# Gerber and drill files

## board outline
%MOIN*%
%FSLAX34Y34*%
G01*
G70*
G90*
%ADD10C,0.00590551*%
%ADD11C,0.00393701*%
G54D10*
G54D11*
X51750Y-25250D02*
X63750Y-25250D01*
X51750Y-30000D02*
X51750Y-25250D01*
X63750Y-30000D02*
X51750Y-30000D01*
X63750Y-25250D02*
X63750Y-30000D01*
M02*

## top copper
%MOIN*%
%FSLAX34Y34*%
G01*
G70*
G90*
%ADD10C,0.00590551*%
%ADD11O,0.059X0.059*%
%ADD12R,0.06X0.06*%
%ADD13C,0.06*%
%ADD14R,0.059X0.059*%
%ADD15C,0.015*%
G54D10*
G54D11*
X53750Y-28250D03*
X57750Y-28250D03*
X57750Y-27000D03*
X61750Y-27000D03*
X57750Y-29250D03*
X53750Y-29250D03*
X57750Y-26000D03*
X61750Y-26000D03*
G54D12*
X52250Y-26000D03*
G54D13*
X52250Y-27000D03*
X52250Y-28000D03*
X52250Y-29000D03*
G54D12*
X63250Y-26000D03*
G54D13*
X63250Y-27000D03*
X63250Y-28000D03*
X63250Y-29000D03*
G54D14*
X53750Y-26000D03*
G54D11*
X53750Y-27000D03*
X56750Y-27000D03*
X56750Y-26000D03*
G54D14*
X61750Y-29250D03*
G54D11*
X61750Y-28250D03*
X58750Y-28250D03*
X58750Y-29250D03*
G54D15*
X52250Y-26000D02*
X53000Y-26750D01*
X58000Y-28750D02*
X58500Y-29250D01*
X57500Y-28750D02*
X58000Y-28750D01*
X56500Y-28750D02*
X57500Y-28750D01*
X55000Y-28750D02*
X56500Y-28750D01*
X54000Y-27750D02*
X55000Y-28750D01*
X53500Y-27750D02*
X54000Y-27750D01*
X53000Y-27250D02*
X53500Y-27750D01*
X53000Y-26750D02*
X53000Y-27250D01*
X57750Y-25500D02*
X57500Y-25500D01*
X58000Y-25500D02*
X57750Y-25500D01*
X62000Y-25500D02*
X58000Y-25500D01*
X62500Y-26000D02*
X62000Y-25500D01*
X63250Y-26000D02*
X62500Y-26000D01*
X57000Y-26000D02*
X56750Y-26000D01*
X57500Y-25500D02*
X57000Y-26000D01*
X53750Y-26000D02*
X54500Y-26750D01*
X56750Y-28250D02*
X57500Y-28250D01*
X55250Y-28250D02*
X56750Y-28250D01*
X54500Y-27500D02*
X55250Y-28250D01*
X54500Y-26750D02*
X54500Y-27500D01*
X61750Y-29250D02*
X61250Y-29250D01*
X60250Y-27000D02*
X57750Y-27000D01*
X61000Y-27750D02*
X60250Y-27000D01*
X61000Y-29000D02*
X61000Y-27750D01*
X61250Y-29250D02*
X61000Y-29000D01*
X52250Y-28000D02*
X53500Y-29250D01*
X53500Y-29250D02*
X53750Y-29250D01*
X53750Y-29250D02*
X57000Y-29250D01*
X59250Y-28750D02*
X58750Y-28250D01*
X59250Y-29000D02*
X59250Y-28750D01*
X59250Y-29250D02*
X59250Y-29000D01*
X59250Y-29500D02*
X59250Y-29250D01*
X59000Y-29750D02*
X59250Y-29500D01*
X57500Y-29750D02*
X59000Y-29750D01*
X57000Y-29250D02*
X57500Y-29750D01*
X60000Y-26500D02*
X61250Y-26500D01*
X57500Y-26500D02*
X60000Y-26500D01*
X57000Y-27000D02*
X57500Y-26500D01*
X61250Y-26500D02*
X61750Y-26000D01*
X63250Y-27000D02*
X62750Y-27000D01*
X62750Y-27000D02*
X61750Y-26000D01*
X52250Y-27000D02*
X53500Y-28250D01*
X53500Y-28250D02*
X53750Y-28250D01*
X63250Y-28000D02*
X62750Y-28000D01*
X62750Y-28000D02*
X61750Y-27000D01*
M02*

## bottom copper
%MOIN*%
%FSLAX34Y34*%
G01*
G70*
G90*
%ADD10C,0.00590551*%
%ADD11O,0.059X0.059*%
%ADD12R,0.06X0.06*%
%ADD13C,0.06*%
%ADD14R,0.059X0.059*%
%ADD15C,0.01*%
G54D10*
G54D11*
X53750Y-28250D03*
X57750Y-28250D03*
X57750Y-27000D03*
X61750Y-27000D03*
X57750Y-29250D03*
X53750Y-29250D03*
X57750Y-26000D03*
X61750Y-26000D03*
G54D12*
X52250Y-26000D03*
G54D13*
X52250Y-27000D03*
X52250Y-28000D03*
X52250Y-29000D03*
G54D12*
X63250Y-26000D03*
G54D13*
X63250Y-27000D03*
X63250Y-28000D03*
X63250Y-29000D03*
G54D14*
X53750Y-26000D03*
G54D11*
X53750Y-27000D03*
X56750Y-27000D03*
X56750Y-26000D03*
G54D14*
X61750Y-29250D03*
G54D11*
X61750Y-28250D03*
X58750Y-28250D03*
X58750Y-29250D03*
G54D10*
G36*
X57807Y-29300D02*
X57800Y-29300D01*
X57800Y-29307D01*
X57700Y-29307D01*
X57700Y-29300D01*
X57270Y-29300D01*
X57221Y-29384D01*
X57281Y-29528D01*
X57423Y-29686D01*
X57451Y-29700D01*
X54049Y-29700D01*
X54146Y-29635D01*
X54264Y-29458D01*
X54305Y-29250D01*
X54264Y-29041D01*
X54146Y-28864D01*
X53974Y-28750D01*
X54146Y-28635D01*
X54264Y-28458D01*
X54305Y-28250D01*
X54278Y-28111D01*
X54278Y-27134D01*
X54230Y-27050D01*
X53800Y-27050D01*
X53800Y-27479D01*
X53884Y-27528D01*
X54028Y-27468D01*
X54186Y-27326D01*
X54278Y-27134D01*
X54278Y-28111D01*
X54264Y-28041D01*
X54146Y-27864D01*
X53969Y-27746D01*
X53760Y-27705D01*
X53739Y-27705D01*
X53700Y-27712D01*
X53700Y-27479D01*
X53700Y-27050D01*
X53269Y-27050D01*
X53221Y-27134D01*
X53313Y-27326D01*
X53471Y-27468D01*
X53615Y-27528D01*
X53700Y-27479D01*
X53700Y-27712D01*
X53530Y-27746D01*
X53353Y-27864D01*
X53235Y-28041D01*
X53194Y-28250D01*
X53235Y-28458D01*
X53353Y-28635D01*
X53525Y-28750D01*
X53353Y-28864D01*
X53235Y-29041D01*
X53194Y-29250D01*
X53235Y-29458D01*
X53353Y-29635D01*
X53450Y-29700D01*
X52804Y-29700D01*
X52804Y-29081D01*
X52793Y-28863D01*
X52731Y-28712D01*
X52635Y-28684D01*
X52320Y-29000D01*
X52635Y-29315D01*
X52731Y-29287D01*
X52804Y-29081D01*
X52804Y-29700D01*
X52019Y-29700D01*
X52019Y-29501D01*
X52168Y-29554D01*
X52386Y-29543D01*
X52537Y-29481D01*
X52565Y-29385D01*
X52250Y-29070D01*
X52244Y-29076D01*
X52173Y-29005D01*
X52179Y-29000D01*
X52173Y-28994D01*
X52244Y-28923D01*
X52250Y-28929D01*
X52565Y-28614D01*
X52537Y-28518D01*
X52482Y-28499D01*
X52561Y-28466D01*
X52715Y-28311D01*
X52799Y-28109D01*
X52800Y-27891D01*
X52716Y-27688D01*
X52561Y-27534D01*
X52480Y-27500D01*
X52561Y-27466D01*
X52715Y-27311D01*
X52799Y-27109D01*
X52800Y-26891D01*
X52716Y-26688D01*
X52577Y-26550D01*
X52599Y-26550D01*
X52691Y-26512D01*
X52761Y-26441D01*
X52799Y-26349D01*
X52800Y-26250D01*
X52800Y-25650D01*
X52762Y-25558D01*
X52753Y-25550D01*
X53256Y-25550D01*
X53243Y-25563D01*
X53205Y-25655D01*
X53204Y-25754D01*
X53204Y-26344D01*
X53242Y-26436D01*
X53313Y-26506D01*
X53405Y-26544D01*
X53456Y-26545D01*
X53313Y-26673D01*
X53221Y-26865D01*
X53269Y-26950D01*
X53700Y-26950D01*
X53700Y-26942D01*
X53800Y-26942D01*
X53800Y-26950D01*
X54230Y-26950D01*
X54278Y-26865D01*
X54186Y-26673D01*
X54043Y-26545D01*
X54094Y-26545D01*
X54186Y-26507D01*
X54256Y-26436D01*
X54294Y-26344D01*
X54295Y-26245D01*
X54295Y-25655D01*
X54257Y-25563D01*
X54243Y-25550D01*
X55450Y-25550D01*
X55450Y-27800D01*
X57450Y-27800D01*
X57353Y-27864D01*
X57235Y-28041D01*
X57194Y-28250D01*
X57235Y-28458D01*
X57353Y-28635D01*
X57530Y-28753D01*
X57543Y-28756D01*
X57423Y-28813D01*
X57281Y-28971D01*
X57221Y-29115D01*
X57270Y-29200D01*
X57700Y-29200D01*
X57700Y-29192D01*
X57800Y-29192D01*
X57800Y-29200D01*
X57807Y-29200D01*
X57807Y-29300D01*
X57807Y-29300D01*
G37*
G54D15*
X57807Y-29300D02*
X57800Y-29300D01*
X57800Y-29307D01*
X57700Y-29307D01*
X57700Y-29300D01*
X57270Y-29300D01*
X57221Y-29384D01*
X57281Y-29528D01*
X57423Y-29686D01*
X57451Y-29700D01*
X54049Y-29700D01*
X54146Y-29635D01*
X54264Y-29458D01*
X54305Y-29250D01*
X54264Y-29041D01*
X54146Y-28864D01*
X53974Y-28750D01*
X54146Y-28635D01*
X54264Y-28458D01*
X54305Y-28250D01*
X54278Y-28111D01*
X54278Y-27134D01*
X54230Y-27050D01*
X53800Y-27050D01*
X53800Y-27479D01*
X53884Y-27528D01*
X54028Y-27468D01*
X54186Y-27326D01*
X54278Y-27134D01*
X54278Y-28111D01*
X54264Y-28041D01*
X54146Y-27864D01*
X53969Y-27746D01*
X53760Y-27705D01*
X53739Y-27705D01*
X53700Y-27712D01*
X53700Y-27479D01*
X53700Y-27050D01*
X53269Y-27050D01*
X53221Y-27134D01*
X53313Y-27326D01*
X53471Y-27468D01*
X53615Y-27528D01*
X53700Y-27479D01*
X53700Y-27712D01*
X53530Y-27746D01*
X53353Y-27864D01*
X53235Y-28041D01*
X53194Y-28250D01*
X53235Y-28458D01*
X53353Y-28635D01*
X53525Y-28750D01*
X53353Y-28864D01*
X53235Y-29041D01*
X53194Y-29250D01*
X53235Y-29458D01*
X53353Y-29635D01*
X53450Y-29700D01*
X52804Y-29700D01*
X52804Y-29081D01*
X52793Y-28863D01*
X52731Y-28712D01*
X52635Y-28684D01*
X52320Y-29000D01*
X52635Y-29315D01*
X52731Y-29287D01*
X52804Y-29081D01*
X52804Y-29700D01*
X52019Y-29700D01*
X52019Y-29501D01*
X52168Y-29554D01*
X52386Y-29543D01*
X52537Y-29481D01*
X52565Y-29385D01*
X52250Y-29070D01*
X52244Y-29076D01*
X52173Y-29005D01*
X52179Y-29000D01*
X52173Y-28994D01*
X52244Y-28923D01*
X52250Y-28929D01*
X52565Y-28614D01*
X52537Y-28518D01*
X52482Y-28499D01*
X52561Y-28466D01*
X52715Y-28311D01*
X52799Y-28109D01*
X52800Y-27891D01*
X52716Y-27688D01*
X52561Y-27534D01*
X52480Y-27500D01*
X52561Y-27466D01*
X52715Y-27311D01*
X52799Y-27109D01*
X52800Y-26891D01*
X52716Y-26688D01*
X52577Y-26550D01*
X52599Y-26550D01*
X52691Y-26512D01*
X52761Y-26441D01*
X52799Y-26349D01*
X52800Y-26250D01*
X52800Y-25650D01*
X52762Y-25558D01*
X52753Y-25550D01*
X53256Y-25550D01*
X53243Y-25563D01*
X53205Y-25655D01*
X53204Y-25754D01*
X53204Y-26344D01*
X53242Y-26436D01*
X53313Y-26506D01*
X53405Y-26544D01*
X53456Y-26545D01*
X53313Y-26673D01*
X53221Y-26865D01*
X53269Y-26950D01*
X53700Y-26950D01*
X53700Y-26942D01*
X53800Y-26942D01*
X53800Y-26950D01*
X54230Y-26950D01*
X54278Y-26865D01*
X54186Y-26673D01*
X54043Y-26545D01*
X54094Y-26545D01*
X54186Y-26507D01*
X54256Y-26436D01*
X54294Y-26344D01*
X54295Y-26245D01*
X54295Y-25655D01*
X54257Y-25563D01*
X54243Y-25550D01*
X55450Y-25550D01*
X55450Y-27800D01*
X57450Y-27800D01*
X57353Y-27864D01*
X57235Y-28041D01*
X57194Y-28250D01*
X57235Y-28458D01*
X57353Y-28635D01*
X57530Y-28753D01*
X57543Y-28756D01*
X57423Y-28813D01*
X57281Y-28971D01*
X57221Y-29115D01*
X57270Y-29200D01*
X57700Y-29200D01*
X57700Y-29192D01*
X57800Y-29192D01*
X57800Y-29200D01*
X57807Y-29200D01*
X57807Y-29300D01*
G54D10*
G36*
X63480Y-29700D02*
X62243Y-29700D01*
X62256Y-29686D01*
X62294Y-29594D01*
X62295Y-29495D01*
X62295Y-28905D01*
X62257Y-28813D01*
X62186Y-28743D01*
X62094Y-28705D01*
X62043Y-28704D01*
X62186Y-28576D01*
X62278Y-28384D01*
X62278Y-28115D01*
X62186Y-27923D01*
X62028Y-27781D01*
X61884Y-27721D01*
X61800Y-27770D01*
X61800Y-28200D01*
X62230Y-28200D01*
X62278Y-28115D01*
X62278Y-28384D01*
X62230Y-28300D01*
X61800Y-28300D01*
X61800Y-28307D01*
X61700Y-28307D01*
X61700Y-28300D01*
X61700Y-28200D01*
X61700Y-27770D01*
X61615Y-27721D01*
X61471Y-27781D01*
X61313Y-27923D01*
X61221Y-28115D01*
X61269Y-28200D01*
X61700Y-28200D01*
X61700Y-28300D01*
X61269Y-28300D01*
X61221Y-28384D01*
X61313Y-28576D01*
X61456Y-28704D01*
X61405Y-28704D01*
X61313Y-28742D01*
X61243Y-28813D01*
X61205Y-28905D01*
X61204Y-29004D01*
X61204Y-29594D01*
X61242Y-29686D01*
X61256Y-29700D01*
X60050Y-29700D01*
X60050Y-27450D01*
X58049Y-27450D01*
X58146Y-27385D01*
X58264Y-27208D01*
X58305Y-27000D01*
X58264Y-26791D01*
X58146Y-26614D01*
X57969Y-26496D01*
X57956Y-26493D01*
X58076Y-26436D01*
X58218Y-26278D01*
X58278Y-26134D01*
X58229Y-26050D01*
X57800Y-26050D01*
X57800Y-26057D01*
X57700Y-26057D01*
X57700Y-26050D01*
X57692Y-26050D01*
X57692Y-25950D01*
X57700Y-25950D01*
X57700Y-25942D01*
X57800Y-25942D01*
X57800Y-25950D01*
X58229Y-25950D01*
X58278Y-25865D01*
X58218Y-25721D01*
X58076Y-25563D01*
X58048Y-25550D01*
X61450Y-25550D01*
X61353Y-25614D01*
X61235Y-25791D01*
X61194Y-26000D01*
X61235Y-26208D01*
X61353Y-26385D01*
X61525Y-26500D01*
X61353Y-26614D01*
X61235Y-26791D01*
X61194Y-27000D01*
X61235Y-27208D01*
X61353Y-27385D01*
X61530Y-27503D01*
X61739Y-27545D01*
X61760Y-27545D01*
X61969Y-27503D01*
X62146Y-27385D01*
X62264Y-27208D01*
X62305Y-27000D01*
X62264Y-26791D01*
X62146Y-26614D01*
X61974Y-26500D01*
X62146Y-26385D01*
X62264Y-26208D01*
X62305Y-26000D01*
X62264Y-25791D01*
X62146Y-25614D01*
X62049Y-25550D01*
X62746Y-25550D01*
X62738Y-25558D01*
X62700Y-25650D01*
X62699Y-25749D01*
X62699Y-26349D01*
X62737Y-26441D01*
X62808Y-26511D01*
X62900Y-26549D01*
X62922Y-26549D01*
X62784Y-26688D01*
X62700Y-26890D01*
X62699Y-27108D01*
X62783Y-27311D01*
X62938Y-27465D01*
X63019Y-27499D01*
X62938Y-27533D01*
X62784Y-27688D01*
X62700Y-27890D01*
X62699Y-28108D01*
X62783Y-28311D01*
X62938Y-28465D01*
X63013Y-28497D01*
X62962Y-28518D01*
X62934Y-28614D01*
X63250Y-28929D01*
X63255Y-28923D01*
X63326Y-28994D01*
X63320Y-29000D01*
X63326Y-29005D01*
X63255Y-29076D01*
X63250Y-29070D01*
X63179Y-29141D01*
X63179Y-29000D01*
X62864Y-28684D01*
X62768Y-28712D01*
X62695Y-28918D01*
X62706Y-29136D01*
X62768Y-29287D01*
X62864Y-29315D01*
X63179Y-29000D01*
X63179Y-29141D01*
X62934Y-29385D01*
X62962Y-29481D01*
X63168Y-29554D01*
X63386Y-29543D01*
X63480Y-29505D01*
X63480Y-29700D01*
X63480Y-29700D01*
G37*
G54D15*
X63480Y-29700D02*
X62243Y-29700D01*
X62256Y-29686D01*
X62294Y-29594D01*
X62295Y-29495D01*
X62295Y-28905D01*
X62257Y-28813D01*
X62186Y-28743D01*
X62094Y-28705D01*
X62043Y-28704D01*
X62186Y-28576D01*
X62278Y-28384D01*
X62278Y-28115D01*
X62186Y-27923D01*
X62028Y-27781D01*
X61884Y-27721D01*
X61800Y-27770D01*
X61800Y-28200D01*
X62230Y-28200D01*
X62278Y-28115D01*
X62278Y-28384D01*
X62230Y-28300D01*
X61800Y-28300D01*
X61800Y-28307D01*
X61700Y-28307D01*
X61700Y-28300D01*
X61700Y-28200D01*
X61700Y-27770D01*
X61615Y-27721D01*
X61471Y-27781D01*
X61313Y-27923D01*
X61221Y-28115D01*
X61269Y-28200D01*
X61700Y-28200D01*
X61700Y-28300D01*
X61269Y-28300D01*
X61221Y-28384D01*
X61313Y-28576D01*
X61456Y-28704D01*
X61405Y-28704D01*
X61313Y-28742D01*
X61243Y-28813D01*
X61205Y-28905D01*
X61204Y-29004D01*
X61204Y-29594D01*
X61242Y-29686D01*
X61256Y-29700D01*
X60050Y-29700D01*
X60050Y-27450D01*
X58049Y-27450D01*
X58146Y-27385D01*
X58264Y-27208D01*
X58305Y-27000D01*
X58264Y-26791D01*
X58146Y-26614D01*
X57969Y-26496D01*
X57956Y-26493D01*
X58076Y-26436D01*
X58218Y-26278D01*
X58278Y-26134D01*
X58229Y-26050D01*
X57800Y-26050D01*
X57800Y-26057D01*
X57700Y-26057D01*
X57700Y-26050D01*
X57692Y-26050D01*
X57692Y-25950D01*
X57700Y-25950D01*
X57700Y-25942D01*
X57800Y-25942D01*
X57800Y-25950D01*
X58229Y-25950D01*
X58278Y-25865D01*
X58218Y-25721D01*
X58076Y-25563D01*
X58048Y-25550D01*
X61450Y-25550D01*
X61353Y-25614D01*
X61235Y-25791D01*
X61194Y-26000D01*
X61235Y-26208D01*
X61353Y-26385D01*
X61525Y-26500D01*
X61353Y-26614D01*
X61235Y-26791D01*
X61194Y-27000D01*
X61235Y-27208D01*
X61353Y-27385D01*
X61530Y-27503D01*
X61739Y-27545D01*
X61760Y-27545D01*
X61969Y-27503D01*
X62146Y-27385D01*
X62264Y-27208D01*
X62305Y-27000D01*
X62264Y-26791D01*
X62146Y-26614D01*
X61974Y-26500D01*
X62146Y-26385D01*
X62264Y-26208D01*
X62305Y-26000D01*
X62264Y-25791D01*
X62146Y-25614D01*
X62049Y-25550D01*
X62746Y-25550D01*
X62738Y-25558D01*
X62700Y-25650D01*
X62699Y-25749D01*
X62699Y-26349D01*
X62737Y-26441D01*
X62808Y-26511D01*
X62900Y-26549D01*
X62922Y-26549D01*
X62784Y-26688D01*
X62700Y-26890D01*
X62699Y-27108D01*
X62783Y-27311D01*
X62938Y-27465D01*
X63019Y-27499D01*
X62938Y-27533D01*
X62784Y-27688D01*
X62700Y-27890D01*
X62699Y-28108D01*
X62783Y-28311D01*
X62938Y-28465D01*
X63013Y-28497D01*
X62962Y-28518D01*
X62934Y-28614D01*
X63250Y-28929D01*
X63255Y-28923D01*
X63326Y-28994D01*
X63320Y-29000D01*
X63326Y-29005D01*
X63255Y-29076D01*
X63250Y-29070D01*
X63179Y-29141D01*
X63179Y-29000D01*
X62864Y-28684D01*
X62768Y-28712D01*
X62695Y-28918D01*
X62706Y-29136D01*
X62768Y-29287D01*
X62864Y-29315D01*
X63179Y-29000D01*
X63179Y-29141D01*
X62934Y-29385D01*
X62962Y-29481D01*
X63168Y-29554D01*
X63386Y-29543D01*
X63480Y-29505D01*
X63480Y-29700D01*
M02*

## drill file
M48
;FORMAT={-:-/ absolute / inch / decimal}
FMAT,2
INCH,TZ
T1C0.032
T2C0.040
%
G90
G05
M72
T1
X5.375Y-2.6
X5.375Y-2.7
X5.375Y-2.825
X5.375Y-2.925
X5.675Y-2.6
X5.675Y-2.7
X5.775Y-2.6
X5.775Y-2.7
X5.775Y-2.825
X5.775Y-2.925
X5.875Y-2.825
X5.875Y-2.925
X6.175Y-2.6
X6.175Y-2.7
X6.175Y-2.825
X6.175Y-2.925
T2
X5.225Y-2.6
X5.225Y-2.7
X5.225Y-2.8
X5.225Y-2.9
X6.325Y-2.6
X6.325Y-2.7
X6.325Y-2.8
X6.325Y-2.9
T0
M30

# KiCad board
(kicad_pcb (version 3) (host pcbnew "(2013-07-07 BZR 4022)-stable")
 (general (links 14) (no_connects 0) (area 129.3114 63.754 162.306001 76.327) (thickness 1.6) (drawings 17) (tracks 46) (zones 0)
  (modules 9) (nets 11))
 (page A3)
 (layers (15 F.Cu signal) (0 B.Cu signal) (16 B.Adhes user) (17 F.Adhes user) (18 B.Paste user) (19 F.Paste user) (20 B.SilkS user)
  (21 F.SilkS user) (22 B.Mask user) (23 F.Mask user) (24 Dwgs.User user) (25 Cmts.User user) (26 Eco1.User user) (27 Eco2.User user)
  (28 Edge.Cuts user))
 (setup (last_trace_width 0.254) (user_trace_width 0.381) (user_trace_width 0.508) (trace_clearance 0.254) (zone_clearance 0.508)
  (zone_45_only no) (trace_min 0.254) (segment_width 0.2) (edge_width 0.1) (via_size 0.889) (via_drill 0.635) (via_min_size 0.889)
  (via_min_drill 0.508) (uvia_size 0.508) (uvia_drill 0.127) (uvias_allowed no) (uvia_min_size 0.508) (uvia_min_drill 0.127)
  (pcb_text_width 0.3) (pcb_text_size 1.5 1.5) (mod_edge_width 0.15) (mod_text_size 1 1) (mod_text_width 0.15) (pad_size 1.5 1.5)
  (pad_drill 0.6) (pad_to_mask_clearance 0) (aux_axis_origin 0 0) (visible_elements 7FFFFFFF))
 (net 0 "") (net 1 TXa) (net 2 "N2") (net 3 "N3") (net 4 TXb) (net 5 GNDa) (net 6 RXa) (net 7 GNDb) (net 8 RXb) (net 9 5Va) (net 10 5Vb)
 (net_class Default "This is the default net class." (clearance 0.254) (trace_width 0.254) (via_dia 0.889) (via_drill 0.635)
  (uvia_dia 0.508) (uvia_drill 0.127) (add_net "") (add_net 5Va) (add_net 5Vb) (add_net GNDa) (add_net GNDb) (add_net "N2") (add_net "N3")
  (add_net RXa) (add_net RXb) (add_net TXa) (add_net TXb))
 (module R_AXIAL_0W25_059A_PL (layer F.Cu) (at 136.525 71.755) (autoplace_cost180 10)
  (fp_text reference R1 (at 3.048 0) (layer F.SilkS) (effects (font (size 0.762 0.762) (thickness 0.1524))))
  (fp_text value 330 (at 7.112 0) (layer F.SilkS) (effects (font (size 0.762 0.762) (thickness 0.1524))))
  (pad 1 thru_hole oval (at 0 0) (size 1.4986 1.4986) (drill 0.8128) (layers *.Cu *.Mask F.SilkS) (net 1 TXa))
  (pad 2 thru_hole oval (at 10.16 0) (size 1.4986 1.4986) (drill 0.8128) (layers *.Cu *.Mask F.SilkS) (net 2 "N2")))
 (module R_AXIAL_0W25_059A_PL (layer F.Cu) (at 146.685 68.58) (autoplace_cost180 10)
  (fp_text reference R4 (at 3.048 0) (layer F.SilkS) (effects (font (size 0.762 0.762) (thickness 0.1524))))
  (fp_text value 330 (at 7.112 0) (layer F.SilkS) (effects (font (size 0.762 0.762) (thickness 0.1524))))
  (pad 1 thru_hole oval (at 0 0) (size 1.4986 1.4986) (drill 0.8128) (layers *.Cu *.Mask F.SilkS) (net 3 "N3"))
  (pad 2 thru_hole oval (at 10.16 0) (size 1.4986 1.4986) (drill 0.8128) (layers *.Cu *.Mask F.SilkS) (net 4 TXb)))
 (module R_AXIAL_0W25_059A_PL (layer F.Cu) (at 146.685 74.295 180) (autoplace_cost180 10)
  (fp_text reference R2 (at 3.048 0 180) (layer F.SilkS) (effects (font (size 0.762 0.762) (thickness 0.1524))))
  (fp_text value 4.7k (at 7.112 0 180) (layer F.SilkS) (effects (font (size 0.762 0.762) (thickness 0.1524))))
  (pad 1 thru_hole oval (at 0 0 180) (size 1.4986 1.4986) (drill 0.8128) (layers *.Cu *.Mask F.SilkS) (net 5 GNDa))
  (pad 2 thru_hole oval (at 10.16 0 180) (size 1.4986 1.4986) (drill 0.8128) (layers *.Cu *.Mask F.SilkS) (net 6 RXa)))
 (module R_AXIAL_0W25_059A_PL (layer F.Cu) (at 146.685 66.04) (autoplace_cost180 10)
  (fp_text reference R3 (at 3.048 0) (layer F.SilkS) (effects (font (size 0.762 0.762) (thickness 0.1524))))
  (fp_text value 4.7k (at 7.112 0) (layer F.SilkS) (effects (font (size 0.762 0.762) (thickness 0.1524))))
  (pad 1 thru_hole oval (at 0 0) (size 1.4986 1.4986) (drill 0.8128) (layers *.Cu *.Mask F.SilkS) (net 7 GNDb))
  (pad 2 thru_hole oval (at 10.16 0) (size 1.4986 1.4986) (drill 0.8128) (layers *.Cu *.Mask F.SilkS) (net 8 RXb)))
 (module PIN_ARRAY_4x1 (layer F.Cu) (at 132.715 69.85 270)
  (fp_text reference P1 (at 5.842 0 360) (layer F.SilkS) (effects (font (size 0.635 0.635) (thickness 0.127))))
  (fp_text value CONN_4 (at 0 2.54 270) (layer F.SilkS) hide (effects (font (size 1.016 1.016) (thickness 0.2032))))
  (pad 1 thru_hole rect (at -3.81 0 270) (size 1.524 1.524) (drill 1.016) (layers *.Cu *.Mask F.SilkS) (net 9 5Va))
  (pad 2 thru_hole circle (at -1.27 0 270) (size 1.524 1.524) (drill 1.016) (layers *.Cu *.Mask F.SilkS) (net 1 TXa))
  (pad 3 thru_hole circle (at 1.27 0 270) (size 1.524 1.524) (drill 1.016) (layers *.Cu *.Mask F.SilkS) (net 6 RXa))
  (pad 4 thru_hole circle (at 3.81 0 270) (size 1.524 1.524) (drill 1.016) (layers *.Cu *.Mask F.SilkS) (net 5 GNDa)))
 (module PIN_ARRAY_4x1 (layer F.Cu) (at 160.655 69.85 270)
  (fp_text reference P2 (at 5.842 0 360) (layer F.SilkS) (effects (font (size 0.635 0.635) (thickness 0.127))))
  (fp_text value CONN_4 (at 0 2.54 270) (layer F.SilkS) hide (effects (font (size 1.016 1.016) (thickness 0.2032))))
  (pad 1 thru_hole rect (at -3.81 0 270) (size 1.524 1.524) (drill 1.016) (layers *.Cu *.Mask F.SilkS) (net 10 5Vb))
  (pad 2 thru_hole circle (at -1.27 0 270) (size 1.524 1.524) (drill 1.016) (layers *.Cu *.Mask F.SilkS) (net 8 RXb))
  (pad 3 thru_hole circle (at 1.27 0 270) (size 1.524 1.524) (drill 1.016) (layers *.Cu *.Mask F.SilkS) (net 4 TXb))
  (pad 4 thru_hole circle (at 3.81 0 270) (size 1.524 1.524) (drill 1.016) (layers *.Cu *.Mask F.SilkS) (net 7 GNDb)))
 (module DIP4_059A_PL (layer F.Cu) (at 140.335 67.31 270)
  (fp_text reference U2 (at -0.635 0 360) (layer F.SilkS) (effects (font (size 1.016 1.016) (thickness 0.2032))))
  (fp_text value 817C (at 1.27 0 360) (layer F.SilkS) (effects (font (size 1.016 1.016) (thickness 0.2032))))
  (pad 1 thru_hole rect (at -1.27 3.81 270) (size 1.4986 1.4986) (drill 0.8128) (layers *.Cu *.Mask F.SilkS) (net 2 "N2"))
  (pad 2 thru_hole oval (at 1.27 3.81 270) (size 1.4986 1.4986) (drill 0.8128) (layers *.Cu *.Mask F.SilkS) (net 5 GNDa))
  (pad 3 thru_hole oval (at 1.27 -3.81 270) (size 1.4986 1.4986) (drill 0.8128) (layers *.Cu *.Mask F.SilkS) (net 8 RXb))
  (pad 4 thru_hole oval (at -1.27 -3.81 270) (size 1.4986 1.4986) (drill 0.8128) (layers *.Cu *.Mask F.SilkS) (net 10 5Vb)))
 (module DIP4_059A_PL (layer F.Cu) (at 153.035 73.025 90)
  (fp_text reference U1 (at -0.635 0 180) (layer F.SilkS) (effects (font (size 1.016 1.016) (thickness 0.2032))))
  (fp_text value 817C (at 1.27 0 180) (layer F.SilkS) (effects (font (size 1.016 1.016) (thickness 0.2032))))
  (pad 1 thru_hole rect (at -1.27 3.81 90) (size 1.4986 1.4986) (drill 0.8128) (layers *.Cu *.Mask F.SilkS) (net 3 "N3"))
  (pad 2 thru_hole oval (at 1.27 3.81 90) (size 1.4986 1.4986) (drill 0.8128) (layers *.Cu *.Mask F.SilkS) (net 7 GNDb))
  (pad 3 thru_hole oval (at 1.27 -3.81 90) (size 1.4986 1.4986) (drill 0.8128) (layers *.Cu *.Mask F.SilkS) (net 6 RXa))
  (pad 4 thru_hole oval (at -1.27 -3.81 90) (size 1.4986 1.4986) (drill 0.8128) (layers *.Cu *.Mask F.SilkS) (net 9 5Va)))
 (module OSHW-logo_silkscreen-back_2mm (layer F.Cu) (at 139.065 74.295 90)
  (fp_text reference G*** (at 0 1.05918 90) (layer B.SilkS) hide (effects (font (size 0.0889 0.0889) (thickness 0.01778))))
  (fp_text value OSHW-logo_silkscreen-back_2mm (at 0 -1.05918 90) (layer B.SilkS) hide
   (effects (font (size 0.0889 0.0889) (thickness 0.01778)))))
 (gr_line (start 131.445 64.135) (end 161.925 64.135) (angle 90) (layer Edge.Cuts) (width 0.1))
 (gr_line (start 131.445 76.2) (end 131.445 64.135) (angle 90) (layer Edge.Cuts) (width 0.1))
 (gr_line (start 161.925 76.2) (end 131.445 76.2) (angle 90) (layer Edge.Cuts) (width 0.1))
 (gr_line (start 161.925 64.135) (end 161.925 76.2) (angle 90) (layer Edge.Cuts) (width 0.1))
 (segment (start 132.715 66.04) (end 134.62 67.945) (width 0.381) (layer F.Cu) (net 9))
 (segment (start 147.32 73.025) (end 148.59 74.295) (width 0.381) (layer F.Cu) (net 9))
 (segment (start 146.05 73.025) (end 147.32 73.025) (width 0.381) (layer F.Cu) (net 9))
 (segment (start 143.51 73.025) (end 146.05 73.025) (width 0.381) (layer F.Cu) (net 9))
 (segment (start 139.7 73.025) (end 143.51 73.025) (width 0.381) (layer F.Cu) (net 9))
 (segment (start 137.16 70.485) (end 139.7 73.025) (width 0.381) (layer F.Cu) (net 9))
 (segment (start 135.89 70.485) (end 137.16 70.485) (width 0.381) (layer F.Cu) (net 9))
 (segment (start 134.62 69.215) (end 135.89 70.485) (width 0.381) (layer F.Cu) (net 9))
 (segment (start 134.62 67.945) (end 134.62 69.215) (width 0.381) (layer F.Cu) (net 9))
 (segment (start 146.685 64.77) (end 146.05 64.77) (width 0.381) (layer F.Cu) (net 10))
 (segment (start 147.32 64.77) (end 146.685 64.77) (width 0.381) (layer F.Cu) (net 10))
 (segment (start 157.48 64.77) (end 147.32 64.77) (width 0.381) (layer F.Cu) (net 10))
 (segment (start 158.75 66.04) (end 157.48 64.77) (width 0.381) (layer F.Cu) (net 10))
 (segment (start 160.655 66.04) (end 158.75 66.04) (width 0.381) (layer F.Cu) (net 10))
 (segment (start 144.78 66.04) (end 144.145 66.04) (width 0.381) (layer F.Cu) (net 10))
 (segment (start 146.05 64.77) (end 144.78 66.04) (width 0.381) (layer F.Cu) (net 10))
 (segment (start 136.525 66.04) (end 138.43 67.945) (width 0.381) (layer F.Cu) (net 2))
 (segment (start 144.145 71.755) (end 146.05 71.755) (width 0.381) (layer F.Cu) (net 2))
 (segment (start 140.335 71.755) (end 144.145 71.755) (width 0.381) (layer F.Cu) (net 2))
 (segment (start 138.43 69.85) (end 140.335 71.755) (width 0.381) (layer F.Cu) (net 2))
 (segment (start 138.43 67.945) (end 138.43 69.85) (width 0.381) (layer F.Cu) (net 2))
 (segment (start 156.845 74.295) (end 155.575 74.295) (width 0.381) (layer F.Cu) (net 3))
 (segment (start 153.035 68.58) (end 146.685 68.58) (width 0.381) (layer F.Cu) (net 3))
 (segment (start 154.94 70.485) (end 153.035 68.58) (width 0.381) (layer F.Cu) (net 3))
 (segment (start 154.94 73.66) (end 154.94 70.485) (width 0.381) (layer F.Cu) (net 3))
 (segment (start 155.575 74.295) (end 154.94 73.66) (width 0.381) (layer F.Cu) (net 3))
 (segment (start 132.715 71.12) (end 135.89 74.295) (width 0.381) (layer F.Cu) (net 6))
 (segment (start 135.89 74.295) (end 136.525 74.295) (width 0.381) (layer F.Cu) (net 6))
 (segment (start 136.525 74.295) (end 144.78 74.295) (width 0.381) (layer F.Cu) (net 6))
 (segment (start 150.495 73.025) (end 149.225 71.755) (width 0.381) (layer F.Cu) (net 6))
 (segment (start 150.495 73.66) (end 150.495 73.025) (width 0.381) (layer F.Cu) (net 6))
 (segment (start 150.495 74.295) (end 150.495 73.66) (width 0.381) (layer F.Cu) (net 6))
 (segment (start 150.495 74.93) (end 150.495 74.295) (width 0.381) (layer F.Cu) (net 6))
 (segment (start 149.86 75.565) (end 150.495 74.93) (width 0.381) (layer F.Cu) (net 6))
 (segment (start 146.05 75.565) (end 149.86 75.565) (width 0.381) (layer F.Cu) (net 6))
 (segment (start 144.78 74.295) (end 146.05 75.565) (width 0.381) (layer F.Cu) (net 6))
 (segment (start 152.4 67.31) (end 155.575 67.31) (width 0.381) (layer F.Cu) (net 8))
 (segment (start 146.05 67.31) (end 152.4 67.31) (width 0.381) (layer F.Cu) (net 8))
 (segment (start 144.78 68.58) (end 146.05 67.31) (width 0.381) (layer F.Cu) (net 8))
 (segment (start 155.575 67.31) (end 156.845 66.04) (width 0.381) (layer F.Cu) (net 8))
 (segment (start 160.655 68.58) (end 159.385 68.58) (width 0.381) (layer F.Cu) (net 8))
 (segment (start 159.385 68.58) (end 156.845 66.04) (width 0.381) (layer F.Cu) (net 8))
 (segment (start 132.715 68.58) (end 135.89 71.755) (width 0.381) (layer F.Cu) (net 1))
 (segment (start 135.89 71.755) (end 136.525 71.755) (width 0.381) (layer F.Cu) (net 1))
 (segment (start 160.655 71.12) (end 159.385 71.12) (width 0.381) (layer F.Cu) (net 4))
 (segment (start 159.385 71.12) (end 156.845 68.58) (width 0.381) (layer F.Cu) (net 4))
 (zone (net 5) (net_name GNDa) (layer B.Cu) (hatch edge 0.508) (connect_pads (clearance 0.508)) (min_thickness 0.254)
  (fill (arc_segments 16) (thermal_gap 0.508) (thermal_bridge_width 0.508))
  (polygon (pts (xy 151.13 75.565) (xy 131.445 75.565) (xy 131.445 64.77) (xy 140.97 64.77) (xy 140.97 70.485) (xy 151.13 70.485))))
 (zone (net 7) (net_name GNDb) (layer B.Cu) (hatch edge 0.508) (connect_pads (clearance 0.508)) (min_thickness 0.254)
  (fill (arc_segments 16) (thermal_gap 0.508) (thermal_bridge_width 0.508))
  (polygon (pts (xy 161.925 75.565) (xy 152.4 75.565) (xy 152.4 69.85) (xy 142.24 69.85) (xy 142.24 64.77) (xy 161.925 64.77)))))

